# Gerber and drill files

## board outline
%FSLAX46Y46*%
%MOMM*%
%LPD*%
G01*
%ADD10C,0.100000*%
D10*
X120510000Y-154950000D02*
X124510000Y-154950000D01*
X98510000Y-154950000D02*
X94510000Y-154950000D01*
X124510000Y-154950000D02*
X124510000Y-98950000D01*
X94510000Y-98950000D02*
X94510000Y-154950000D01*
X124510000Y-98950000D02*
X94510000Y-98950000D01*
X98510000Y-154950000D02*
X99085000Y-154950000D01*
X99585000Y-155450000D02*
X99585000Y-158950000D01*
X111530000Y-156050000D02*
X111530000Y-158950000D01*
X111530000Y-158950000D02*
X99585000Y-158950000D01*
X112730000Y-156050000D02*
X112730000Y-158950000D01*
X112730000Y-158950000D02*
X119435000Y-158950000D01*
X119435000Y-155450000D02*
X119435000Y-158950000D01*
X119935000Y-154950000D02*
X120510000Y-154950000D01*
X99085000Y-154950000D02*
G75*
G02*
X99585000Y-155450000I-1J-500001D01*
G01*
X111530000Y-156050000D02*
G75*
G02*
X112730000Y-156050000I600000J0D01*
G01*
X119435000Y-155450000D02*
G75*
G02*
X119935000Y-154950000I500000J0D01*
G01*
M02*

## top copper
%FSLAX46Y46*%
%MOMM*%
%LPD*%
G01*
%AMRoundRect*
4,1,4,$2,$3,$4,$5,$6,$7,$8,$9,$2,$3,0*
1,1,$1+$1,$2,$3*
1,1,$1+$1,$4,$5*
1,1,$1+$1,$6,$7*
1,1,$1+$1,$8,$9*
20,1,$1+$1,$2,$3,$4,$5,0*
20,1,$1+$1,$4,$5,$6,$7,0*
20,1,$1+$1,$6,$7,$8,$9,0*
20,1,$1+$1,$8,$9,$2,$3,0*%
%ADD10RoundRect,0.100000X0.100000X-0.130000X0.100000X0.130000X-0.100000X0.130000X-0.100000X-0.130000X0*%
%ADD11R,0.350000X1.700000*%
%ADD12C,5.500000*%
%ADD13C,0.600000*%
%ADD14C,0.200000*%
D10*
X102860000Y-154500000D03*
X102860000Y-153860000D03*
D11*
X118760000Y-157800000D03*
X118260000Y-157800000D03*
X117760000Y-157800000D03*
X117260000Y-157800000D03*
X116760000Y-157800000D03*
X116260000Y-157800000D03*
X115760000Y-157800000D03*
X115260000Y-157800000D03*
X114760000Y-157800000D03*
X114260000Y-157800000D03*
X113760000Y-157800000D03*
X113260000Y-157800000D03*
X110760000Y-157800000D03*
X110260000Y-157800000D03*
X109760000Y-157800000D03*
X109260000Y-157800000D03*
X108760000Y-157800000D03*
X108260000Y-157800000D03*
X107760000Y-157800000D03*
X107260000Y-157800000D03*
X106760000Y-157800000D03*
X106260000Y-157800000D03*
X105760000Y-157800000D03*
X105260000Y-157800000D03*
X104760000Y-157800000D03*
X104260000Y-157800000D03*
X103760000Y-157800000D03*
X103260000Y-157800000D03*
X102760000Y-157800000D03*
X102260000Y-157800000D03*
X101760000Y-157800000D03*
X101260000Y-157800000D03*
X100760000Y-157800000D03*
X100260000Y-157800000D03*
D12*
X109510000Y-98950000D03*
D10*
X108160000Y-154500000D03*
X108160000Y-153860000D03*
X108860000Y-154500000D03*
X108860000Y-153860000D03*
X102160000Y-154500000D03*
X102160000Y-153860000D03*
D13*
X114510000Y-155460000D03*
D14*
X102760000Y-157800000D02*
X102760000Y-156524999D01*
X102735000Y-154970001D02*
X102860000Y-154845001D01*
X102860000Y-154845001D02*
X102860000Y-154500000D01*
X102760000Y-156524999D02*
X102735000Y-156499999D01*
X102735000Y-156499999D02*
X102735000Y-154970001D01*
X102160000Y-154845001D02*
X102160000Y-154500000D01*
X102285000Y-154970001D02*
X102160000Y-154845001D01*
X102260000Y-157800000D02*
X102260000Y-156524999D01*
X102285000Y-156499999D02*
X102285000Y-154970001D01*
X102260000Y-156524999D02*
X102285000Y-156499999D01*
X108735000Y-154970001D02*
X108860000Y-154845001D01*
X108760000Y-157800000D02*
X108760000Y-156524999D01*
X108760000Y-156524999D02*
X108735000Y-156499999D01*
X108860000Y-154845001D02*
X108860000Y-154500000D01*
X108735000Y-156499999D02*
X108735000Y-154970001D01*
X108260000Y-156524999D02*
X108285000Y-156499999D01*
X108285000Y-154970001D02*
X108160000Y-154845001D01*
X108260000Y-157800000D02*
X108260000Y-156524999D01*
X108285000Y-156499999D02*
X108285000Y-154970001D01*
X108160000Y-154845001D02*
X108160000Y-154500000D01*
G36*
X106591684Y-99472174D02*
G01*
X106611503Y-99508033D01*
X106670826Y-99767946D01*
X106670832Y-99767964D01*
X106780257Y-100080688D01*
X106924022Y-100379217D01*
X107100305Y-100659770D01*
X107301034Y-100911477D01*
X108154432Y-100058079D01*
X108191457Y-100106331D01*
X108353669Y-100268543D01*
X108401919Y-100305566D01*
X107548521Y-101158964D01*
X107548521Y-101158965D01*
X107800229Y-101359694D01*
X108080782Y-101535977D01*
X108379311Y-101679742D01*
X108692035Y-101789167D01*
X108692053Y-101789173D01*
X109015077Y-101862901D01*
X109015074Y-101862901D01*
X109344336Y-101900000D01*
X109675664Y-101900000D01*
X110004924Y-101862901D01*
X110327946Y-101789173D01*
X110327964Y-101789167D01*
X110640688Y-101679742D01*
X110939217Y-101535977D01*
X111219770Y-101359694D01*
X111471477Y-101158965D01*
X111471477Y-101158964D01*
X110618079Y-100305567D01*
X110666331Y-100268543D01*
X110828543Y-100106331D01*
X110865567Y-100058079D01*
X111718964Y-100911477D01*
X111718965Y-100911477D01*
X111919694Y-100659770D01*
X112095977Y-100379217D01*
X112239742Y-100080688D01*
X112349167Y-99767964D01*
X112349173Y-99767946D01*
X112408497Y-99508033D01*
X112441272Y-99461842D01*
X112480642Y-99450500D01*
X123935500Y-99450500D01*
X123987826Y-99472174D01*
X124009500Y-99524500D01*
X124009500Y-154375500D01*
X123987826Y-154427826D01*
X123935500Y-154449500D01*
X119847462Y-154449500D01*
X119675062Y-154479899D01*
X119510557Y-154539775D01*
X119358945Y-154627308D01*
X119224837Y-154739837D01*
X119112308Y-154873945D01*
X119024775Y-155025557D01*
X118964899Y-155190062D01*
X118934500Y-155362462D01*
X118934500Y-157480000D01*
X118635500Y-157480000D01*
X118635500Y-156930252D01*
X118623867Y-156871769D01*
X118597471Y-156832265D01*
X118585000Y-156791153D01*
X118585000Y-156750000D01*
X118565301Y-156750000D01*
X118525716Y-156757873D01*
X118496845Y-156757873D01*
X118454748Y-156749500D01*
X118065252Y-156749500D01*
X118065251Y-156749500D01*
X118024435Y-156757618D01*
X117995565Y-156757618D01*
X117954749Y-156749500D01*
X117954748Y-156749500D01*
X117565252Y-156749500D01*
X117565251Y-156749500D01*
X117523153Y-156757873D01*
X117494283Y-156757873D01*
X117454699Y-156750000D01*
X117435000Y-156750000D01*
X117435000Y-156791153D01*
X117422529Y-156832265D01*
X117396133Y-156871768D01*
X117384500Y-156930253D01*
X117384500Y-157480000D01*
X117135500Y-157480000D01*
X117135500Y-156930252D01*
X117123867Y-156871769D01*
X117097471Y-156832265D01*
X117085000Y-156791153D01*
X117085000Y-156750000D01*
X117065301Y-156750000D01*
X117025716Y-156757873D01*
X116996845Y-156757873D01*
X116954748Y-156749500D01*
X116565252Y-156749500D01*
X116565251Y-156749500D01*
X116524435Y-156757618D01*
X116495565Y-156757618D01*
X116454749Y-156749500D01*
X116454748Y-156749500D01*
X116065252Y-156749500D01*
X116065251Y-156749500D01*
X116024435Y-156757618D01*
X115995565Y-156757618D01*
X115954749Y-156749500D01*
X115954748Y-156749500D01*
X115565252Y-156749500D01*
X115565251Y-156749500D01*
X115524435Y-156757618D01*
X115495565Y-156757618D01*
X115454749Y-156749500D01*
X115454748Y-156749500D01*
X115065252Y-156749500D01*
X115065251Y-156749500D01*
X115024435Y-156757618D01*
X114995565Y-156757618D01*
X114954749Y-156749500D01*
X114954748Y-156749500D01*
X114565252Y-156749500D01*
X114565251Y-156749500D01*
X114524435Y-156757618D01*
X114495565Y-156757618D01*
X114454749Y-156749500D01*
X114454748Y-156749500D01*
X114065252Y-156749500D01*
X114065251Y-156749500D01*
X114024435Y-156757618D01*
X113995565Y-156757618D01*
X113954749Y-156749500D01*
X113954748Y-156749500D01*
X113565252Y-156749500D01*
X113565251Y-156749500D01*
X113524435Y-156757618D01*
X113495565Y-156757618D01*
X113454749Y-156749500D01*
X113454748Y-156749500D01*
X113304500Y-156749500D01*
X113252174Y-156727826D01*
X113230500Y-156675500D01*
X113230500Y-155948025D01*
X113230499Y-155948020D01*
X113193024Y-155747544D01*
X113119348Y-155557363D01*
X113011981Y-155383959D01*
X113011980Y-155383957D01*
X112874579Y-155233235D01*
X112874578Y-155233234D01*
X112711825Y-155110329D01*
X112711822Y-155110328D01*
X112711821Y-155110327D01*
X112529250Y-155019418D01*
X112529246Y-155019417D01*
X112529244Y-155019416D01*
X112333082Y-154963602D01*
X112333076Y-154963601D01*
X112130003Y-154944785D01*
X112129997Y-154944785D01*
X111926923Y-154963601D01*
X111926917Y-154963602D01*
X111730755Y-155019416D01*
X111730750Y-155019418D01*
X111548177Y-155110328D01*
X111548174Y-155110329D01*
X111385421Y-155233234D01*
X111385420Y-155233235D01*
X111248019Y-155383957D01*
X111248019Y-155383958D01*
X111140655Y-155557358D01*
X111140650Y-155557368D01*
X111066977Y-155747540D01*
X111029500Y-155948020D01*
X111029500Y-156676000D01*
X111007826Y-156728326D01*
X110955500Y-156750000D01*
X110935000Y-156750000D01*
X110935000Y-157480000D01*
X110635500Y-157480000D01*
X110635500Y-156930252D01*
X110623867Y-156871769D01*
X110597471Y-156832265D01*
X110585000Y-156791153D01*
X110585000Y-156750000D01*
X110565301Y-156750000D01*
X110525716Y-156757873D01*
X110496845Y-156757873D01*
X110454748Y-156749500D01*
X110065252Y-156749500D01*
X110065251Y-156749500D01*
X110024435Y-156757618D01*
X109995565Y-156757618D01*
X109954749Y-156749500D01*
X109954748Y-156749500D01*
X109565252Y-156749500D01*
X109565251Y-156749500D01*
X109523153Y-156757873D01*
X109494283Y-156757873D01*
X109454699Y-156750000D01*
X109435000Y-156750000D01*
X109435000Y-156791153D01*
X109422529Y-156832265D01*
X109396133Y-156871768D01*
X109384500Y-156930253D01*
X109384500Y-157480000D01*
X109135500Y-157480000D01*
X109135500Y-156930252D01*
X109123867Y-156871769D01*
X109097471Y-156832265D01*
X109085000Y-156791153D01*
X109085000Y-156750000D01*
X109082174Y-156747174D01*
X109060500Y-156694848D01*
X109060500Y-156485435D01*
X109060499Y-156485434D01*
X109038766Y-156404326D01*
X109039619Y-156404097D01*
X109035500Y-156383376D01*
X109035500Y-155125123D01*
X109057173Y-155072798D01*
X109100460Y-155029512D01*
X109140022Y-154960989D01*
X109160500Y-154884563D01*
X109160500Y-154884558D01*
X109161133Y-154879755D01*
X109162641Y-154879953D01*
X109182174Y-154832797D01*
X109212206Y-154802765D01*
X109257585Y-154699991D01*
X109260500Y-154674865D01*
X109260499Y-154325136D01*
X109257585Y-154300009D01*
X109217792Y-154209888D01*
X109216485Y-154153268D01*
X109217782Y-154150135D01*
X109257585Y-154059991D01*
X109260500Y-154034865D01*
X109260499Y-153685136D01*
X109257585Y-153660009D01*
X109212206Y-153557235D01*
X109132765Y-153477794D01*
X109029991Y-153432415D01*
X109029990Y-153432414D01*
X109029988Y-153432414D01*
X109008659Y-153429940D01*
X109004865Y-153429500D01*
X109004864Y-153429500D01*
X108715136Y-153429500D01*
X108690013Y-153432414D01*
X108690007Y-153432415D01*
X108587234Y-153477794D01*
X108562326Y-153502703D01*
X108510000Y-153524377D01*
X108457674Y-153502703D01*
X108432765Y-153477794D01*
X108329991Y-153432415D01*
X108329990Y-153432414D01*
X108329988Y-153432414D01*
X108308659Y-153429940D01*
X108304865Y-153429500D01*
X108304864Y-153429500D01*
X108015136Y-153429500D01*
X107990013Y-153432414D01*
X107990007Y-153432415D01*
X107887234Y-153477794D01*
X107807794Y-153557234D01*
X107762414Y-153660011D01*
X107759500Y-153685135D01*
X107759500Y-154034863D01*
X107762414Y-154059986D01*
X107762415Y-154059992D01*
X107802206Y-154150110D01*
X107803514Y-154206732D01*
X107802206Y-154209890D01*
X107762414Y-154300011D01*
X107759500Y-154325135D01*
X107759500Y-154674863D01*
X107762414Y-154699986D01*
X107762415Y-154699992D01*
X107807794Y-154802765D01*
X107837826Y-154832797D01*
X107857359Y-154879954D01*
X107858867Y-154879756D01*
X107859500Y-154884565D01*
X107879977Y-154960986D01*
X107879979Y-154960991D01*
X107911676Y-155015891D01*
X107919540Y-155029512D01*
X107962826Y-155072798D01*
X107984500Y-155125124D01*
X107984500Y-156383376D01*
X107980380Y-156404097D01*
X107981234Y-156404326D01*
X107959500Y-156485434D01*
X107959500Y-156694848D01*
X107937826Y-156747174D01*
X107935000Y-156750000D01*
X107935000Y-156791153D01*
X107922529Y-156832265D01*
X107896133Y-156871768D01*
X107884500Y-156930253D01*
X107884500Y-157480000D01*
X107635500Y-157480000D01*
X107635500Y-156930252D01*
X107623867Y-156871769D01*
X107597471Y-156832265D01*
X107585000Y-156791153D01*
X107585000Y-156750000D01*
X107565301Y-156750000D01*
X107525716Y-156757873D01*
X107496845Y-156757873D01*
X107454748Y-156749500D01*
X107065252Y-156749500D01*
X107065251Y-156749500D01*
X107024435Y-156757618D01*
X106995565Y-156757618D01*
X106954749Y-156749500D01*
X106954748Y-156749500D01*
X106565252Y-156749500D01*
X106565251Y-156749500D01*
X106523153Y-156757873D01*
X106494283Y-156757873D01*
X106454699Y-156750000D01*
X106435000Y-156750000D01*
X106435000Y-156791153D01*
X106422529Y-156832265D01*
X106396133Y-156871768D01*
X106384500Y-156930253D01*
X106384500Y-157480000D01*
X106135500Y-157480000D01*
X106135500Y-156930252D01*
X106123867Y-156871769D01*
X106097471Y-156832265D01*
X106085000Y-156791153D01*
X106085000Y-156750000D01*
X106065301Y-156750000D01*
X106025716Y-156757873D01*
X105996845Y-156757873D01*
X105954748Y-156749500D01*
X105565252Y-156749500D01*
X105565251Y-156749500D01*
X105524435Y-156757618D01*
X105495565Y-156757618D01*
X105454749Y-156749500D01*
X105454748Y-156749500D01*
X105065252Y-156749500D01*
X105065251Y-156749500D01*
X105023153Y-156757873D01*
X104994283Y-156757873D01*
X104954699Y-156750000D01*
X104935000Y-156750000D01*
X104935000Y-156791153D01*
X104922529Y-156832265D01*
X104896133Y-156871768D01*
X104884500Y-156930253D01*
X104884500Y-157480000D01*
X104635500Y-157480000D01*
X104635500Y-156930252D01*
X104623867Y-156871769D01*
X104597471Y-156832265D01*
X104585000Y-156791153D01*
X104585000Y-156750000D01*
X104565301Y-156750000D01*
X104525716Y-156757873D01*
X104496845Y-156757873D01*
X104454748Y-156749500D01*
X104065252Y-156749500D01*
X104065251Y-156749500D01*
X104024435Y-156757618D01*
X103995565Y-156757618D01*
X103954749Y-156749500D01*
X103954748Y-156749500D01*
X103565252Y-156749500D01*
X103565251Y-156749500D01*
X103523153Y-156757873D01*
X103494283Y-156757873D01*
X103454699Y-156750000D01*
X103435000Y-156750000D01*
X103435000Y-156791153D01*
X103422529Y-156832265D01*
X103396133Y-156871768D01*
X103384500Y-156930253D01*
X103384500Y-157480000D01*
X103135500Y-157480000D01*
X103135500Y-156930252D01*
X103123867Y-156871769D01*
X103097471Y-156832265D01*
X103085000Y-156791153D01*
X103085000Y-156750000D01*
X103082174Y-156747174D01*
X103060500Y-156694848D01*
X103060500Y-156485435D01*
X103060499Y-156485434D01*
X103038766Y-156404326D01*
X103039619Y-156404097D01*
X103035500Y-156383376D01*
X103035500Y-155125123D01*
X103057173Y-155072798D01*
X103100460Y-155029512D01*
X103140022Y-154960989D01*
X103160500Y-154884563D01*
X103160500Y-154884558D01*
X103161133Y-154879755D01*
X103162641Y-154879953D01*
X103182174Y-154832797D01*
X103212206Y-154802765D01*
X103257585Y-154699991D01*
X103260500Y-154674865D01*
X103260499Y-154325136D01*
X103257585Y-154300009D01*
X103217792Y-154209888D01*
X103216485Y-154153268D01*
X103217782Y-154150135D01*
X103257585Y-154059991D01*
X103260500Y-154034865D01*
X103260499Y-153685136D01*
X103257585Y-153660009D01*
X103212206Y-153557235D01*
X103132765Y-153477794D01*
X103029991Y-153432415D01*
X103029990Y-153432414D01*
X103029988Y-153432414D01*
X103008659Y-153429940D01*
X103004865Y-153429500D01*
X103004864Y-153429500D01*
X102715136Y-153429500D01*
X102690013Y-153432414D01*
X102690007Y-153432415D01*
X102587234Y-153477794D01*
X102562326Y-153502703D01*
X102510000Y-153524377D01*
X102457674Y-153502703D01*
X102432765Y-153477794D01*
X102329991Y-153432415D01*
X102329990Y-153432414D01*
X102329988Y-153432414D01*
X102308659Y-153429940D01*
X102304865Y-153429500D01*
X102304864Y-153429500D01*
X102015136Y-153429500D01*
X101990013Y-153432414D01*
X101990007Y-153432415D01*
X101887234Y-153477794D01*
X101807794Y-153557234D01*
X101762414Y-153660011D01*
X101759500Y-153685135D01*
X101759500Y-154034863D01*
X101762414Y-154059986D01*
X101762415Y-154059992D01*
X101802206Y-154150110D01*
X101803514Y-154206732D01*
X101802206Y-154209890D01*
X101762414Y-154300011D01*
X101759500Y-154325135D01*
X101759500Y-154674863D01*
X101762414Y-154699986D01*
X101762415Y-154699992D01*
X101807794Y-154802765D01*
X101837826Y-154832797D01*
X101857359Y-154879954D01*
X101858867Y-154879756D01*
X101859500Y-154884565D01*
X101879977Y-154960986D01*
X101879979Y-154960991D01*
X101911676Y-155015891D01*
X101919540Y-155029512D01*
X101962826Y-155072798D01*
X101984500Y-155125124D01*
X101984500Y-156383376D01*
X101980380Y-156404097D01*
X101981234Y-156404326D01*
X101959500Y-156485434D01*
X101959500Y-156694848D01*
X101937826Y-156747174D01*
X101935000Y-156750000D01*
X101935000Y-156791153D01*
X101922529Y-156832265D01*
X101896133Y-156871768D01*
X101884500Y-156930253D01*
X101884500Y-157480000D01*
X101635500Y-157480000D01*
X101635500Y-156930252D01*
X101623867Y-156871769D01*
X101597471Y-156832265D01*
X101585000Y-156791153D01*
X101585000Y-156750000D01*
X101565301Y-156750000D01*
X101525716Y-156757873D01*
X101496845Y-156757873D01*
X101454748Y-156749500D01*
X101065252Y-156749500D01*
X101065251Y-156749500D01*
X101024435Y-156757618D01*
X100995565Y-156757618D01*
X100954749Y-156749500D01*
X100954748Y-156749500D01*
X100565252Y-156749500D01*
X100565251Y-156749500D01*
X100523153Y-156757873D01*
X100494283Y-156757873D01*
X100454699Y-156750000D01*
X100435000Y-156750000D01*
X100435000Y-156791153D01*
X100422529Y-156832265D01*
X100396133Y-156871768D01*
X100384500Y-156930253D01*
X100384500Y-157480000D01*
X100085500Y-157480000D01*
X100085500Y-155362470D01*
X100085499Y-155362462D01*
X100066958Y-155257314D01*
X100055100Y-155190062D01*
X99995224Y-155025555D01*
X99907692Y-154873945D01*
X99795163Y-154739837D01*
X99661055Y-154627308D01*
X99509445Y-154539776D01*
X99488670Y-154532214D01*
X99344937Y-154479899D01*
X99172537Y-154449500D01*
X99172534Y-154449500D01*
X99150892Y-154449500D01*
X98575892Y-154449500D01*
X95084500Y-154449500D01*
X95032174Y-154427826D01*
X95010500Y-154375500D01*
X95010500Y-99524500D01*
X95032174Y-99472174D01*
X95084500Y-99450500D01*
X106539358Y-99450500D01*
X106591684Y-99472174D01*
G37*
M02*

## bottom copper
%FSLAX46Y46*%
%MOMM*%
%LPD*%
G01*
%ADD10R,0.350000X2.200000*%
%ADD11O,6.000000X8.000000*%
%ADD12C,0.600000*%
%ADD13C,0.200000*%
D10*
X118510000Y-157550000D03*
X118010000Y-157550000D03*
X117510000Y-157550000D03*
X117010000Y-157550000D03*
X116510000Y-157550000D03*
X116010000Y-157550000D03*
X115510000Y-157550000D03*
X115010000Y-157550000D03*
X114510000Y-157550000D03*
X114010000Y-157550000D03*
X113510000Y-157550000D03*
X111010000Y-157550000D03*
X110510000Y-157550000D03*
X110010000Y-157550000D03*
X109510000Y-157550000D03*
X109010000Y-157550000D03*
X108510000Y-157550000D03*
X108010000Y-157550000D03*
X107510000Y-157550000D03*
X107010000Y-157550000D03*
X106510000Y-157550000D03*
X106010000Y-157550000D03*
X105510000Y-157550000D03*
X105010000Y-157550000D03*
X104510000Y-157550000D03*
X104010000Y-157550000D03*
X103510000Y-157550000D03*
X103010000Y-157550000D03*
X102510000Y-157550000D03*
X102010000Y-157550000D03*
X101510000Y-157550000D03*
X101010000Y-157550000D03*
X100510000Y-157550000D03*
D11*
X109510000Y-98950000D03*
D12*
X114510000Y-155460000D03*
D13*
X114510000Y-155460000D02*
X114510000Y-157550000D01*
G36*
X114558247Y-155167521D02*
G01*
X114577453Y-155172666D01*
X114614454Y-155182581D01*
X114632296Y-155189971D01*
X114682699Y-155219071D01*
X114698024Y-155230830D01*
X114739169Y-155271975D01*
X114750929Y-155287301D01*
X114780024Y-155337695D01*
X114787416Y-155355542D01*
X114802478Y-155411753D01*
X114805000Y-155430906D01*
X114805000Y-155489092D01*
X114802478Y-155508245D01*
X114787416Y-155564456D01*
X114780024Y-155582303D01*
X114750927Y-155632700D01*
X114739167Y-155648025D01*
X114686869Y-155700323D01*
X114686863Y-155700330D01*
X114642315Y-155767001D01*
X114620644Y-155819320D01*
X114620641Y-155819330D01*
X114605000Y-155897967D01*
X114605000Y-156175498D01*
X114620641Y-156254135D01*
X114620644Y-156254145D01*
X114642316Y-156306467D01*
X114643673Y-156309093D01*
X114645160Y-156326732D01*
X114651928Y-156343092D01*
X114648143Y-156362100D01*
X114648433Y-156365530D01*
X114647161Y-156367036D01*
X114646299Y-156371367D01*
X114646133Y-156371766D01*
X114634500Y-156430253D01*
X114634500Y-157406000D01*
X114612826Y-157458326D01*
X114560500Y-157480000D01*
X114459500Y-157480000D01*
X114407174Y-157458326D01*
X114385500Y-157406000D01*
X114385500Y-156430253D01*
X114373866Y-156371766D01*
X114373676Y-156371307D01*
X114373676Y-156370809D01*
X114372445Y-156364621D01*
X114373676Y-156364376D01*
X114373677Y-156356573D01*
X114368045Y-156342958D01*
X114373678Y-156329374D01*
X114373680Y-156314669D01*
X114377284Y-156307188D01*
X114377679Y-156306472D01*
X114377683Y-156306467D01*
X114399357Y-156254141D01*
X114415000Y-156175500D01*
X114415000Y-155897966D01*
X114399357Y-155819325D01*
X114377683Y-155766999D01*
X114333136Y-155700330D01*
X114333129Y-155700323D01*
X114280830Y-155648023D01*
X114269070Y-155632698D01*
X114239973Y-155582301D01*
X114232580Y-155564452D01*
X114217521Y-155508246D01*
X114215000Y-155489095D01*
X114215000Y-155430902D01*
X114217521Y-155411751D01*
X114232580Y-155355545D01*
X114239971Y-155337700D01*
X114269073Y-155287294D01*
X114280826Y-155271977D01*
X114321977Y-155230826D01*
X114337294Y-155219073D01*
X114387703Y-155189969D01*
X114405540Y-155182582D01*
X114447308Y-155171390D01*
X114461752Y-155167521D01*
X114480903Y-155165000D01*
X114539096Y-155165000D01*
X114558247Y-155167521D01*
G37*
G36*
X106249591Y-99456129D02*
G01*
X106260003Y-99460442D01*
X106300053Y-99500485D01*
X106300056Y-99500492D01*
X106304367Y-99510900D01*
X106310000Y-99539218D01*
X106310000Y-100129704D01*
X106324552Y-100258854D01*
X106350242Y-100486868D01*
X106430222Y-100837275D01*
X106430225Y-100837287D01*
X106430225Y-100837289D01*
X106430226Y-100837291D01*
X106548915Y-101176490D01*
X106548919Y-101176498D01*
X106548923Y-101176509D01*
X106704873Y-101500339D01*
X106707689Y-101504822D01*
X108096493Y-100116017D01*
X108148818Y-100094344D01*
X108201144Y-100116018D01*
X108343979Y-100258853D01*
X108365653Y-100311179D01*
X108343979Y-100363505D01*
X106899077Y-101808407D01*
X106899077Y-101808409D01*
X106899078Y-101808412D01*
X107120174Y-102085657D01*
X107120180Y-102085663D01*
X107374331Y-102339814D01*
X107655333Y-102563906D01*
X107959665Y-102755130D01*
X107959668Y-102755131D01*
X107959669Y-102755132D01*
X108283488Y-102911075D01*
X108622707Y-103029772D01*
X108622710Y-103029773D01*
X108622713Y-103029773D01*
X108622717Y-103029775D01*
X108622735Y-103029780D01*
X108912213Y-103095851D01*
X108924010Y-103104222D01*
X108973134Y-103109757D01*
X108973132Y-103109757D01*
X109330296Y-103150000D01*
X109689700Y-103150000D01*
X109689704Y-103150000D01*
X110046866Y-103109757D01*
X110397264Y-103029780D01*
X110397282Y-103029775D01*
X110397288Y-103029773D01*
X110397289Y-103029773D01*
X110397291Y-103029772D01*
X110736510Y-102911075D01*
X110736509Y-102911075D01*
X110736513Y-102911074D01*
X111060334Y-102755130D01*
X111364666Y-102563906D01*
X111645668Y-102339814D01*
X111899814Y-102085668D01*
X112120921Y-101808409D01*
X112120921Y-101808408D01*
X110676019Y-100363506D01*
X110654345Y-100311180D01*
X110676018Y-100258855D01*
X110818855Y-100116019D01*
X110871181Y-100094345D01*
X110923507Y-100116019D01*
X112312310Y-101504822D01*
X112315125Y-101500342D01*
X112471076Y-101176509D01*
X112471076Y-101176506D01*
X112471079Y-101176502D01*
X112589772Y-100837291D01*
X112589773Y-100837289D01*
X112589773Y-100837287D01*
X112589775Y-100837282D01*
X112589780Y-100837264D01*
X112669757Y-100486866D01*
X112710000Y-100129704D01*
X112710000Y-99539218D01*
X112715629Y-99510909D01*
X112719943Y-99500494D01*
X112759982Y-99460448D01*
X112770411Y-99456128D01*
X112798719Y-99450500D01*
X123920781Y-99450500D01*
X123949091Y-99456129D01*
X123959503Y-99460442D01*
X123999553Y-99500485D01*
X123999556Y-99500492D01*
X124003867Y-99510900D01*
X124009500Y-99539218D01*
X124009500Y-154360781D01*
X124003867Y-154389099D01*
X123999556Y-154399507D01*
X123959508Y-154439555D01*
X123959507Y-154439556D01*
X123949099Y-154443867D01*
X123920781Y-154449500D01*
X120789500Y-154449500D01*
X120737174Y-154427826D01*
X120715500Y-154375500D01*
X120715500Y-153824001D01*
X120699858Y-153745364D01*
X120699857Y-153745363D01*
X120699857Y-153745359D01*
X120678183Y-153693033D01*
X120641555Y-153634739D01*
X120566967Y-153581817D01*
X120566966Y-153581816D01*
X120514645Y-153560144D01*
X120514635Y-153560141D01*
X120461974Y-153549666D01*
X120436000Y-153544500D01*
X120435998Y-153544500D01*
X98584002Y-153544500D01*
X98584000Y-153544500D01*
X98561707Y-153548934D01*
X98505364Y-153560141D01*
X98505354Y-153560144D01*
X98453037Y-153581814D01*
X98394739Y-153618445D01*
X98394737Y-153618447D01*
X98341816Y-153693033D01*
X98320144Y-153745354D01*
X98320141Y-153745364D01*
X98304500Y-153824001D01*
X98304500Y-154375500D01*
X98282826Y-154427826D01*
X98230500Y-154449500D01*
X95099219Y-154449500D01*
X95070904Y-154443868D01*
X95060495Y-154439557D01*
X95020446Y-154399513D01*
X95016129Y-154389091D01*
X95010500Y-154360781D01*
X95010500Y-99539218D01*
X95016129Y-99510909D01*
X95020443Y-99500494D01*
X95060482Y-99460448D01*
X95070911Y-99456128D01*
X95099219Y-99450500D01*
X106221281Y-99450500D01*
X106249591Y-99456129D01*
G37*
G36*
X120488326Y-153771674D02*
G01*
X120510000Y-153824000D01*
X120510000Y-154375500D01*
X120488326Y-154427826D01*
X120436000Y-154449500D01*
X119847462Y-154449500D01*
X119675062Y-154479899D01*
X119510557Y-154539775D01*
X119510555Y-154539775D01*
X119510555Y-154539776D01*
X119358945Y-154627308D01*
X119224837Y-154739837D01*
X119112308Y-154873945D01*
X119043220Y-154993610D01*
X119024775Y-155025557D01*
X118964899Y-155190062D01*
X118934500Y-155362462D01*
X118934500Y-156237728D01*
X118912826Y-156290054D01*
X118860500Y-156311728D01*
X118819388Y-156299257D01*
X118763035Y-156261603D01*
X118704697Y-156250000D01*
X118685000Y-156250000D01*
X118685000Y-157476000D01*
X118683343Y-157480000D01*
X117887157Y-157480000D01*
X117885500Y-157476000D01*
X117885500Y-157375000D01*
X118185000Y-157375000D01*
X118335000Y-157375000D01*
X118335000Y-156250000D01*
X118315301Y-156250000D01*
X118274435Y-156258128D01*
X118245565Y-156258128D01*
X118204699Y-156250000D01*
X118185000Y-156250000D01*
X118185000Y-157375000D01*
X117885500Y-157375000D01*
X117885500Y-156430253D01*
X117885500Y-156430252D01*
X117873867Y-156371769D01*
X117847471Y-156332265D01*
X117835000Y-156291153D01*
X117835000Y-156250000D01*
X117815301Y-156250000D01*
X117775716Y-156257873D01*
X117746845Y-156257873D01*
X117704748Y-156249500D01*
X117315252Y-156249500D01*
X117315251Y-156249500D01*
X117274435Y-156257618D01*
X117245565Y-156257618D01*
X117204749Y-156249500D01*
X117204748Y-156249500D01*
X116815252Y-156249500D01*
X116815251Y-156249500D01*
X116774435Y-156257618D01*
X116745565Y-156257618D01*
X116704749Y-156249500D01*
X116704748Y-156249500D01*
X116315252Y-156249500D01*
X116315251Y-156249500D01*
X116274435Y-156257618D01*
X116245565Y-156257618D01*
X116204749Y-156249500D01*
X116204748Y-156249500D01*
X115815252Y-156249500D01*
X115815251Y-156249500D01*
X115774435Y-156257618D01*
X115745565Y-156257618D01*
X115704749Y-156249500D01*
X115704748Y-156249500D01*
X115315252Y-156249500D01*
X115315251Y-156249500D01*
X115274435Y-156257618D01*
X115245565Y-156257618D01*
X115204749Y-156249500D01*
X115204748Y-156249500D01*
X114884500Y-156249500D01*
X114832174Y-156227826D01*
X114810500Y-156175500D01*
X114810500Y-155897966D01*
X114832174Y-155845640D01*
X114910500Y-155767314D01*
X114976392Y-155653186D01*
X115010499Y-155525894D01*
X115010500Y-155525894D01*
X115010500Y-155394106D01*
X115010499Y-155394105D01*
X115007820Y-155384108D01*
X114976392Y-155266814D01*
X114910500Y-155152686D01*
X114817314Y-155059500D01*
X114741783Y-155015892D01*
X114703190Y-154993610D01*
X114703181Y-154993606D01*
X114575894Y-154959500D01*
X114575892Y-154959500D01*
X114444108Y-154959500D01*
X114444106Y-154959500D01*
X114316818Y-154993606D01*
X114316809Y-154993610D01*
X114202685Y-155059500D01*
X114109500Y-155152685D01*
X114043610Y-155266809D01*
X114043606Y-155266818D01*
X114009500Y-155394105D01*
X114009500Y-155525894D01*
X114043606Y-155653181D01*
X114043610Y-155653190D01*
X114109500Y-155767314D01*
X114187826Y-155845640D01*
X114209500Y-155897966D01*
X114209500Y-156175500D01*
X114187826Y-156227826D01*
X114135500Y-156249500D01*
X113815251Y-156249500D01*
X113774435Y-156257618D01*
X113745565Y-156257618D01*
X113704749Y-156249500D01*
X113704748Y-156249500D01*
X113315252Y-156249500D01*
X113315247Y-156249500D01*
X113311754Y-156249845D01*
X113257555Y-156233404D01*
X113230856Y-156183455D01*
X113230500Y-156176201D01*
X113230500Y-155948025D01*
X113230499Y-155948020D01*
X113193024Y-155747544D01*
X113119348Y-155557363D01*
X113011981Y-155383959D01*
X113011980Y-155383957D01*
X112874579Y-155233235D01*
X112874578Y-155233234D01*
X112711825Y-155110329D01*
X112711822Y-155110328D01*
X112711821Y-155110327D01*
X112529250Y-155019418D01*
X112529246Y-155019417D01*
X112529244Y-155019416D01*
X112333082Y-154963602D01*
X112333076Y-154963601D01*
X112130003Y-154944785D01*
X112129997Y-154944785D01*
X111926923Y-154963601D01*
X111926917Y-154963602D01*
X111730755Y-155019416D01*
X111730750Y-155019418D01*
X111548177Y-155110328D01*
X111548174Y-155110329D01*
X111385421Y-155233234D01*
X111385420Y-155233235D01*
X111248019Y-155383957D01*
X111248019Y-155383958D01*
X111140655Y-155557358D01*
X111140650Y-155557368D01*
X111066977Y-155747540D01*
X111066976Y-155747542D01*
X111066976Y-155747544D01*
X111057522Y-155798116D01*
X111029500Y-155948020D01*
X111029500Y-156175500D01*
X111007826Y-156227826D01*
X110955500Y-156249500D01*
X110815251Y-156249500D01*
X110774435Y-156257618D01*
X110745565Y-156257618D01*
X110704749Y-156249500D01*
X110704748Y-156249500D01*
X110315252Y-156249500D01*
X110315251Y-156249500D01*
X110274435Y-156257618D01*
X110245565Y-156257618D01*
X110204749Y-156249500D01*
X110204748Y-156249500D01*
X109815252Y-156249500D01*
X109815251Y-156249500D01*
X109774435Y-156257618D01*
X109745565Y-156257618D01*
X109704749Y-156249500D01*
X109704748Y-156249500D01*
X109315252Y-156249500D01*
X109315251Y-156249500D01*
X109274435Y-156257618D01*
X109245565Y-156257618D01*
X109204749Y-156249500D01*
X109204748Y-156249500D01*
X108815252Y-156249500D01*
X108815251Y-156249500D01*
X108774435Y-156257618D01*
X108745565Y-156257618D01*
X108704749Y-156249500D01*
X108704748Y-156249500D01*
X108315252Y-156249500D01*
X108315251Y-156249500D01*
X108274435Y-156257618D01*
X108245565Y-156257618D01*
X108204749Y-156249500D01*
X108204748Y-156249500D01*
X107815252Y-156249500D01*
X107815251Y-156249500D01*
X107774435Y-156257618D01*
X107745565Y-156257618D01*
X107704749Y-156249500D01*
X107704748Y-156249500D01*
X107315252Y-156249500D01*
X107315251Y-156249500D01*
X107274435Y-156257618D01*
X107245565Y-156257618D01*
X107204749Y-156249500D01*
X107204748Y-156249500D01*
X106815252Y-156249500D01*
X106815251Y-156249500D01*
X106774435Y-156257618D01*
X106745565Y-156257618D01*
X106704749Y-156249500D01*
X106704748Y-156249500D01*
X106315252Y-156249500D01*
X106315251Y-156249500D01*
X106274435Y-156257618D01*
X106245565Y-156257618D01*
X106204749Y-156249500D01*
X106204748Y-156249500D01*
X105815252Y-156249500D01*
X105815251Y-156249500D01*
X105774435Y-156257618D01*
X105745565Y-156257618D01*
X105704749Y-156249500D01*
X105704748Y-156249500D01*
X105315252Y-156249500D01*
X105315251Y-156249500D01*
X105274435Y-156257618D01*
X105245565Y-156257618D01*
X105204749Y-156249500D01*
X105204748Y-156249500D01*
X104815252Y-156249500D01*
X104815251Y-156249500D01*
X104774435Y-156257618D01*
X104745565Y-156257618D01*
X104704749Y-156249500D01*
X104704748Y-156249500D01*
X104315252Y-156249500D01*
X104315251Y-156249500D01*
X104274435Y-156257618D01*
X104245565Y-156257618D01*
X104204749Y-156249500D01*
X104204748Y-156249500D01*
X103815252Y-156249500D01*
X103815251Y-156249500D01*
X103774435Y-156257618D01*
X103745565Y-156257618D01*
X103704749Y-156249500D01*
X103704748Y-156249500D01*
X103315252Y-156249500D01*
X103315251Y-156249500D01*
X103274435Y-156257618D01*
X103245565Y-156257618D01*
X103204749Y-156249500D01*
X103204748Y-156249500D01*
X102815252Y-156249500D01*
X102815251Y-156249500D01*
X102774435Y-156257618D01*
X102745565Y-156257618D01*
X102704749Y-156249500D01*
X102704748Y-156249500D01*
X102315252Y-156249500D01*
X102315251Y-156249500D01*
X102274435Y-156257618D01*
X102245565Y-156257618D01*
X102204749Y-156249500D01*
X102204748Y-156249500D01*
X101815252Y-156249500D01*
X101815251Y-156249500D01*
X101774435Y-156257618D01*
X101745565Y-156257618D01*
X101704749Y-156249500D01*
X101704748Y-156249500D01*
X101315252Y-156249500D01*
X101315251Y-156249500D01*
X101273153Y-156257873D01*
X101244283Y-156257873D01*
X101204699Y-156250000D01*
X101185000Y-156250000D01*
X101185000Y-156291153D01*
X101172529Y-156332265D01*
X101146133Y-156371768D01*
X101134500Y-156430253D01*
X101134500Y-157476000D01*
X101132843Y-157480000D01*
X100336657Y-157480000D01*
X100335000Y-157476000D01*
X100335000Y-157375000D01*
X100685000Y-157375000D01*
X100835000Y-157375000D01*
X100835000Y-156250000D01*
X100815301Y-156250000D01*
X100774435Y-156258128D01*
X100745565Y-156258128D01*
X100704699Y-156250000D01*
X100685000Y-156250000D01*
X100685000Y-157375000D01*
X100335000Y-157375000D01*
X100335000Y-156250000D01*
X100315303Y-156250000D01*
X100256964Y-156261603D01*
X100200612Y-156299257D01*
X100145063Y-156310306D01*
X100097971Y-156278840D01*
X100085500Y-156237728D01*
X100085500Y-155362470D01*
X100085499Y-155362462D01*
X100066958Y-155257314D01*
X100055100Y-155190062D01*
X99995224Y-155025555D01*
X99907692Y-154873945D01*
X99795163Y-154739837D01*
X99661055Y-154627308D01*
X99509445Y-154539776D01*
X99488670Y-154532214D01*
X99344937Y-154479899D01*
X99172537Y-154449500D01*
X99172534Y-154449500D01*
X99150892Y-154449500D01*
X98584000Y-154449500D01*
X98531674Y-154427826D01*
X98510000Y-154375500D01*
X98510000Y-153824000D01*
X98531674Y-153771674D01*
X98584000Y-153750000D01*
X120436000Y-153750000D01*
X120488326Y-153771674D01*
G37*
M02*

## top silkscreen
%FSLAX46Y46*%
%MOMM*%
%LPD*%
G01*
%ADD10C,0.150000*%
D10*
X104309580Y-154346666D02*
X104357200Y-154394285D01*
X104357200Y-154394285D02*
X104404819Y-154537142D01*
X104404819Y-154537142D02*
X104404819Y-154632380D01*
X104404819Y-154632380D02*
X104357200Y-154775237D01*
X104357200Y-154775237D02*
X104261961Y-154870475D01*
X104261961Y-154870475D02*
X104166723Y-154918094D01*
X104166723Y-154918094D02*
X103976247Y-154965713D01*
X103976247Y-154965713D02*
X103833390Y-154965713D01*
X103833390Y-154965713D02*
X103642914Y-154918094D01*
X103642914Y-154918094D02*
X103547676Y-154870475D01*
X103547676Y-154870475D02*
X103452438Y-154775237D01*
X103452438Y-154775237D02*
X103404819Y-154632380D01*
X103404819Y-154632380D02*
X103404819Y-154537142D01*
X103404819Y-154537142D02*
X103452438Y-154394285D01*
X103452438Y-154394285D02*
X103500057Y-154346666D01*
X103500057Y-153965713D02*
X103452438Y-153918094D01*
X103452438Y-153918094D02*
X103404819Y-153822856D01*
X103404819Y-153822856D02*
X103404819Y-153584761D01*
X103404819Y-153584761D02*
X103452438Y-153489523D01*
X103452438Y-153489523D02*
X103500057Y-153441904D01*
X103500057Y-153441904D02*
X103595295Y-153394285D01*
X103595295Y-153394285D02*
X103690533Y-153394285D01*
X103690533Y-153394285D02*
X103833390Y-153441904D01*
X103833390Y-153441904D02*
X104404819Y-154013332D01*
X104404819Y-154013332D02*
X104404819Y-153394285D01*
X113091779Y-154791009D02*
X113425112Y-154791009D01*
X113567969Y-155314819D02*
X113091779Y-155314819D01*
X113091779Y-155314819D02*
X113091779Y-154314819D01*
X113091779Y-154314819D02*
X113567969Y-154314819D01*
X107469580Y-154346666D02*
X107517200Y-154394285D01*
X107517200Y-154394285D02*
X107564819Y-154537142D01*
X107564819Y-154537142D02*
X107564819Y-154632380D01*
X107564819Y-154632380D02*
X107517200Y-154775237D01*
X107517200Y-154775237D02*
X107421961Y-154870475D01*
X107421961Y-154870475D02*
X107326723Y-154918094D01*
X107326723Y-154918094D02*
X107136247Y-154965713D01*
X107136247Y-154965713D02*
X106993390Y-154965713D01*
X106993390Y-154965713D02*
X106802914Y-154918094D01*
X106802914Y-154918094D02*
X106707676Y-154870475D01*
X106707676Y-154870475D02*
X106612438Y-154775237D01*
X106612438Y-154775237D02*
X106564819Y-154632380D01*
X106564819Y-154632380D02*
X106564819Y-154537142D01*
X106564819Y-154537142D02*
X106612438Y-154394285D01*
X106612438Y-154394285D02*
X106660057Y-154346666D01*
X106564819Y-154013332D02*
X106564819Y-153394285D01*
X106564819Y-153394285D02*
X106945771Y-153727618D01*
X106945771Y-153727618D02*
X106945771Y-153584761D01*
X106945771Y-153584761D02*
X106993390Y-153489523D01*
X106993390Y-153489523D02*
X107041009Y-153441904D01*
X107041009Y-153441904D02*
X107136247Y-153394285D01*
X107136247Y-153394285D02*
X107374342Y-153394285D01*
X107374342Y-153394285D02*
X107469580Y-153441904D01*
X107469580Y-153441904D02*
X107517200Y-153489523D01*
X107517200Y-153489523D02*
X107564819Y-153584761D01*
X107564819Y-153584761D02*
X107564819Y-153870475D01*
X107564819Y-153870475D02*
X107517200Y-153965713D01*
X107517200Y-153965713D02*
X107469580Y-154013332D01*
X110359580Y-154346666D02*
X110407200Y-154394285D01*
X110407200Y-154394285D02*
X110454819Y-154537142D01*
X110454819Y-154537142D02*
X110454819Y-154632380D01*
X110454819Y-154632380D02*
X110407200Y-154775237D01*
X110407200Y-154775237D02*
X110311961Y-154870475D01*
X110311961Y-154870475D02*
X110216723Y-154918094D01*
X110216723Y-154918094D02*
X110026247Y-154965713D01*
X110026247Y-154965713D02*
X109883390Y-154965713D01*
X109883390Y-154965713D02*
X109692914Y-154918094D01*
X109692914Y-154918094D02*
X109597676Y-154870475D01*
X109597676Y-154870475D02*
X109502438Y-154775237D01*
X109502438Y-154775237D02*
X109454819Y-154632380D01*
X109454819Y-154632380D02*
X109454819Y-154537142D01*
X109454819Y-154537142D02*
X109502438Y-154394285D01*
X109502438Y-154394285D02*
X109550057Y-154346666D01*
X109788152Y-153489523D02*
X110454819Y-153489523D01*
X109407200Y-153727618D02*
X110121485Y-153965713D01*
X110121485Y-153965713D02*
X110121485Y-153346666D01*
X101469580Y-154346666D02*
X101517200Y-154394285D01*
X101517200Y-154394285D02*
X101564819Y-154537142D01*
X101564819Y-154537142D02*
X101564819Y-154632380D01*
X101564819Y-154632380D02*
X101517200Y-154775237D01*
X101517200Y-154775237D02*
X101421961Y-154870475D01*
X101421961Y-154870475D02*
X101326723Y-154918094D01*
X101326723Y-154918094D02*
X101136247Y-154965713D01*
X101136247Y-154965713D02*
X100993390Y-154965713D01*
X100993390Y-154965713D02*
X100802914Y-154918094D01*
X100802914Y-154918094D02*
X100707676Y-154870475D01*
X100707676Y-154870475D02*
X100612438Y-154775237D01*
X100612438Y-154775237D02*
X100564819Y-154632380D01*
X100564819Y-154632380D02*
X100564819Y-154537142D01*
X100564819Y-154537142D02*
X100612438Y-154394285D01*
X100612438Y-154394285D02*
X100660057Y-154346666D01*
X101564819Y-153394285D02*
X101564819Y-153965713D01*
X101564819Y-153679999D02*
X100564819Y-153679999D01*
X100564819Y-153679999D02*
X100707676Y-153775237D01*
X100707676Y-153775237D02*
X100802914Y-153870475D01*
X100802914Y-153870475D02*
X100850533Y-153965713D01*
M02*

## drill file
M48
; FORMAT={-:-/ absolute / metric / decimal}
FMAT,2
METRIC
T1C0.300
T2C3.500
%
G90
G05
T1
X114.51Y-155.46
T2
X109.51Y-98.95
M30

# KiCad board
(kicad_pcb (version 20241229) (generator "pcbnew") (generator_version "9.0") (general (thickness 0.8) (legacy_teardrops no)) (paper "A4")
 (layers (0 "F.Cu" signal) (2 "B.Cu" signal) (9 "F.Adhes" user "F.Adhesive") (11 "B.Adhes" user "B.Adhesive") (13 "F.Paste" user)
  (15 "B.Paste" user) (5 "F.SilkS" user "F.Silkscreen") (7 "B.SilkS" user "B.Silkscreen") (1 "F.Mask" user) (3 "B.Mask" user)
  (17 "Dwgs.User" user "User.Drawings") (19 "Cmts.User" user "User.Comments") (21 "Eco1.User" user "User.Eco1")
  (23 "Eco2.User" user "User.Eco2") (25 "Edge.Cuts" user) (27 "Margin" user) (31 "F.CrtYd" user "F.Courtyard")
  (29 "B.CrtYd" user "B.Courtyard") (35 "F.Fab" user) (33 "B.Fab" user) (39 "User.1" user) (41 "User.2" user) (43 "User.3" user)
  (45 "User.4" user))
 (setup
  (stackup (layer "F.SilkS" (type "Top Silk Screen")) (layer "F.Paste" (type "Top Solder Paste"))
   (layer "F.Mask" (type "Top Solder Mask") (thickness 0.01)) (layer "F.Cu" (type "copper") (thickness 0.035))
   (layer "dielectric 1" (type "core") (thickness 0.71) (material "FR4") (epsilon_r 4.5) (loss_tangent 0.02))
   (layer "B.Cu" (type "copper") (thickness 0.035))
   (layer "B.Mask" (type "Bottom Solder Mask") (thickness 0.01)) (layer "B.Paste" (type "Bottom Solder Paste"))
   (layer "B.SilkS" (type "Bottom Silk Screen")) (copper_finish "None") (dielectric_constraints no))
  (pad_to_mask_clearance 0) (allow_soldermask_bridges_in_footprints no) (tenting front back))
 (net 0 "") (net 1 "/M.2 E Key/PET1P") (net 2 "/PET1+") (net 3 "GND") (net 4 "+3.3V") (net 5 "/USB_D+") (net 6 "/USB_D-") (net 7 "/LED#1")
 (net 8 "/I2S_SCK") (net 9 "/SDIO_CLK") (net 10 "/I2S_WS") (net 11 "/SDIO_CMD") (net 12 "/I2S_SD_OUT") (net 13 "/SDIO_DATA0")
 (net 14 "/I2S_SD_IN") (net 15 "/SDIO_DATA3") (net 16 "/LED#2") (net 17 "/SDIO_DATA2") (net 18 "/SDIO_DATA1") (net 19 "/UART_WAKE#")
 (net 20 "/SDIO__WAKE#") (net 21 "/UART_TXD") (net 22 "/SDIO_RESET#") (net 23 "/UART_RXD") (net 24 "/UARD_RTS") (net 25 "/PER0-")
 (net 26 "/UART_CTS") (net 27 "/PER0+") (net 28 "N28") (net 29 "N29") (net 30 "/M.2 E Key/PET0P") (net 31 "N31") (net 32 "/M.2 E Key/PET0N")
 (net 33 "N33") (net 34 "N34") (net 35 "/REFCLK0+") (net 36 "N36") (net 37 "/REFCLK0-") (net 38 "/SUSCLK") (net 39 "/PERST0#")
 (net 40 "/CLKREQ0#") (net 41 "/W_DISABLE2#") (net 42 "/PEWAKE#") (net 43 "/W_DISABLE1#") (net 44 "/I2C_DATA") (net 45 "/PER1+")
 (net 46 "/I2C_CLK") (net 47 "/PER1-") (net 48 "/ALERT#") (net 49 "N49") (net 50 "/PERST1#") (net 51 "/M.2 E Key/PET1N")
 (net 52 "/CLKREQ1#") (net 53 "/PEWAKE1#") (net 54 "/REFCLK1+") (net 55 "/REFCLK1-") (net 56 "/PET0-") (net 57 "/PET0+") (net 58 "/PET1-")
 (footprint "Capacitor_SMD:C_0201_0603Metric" (layer "F.Cu") (at 102.86 154.18 90)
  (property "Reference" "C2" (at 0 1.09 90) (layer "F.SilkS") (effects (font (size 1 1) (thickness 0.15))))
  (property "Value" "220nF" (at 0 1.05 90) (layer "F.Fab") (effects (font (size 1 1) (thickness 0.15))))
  (pad "" smd roundrect (at -0.345 0 90) (size 0.318 0.36) (layers "F.Paste") (roundrect_rratio 0.25))
  (pad "" smd roundrect (at 0.345 0 90) (size 0.318 0.36) (layers "F.Paste") (roundrect_rratio 0.25))
  (pad "1" smd roundrect (at -0.32 0 90) (size 0.46 0.4) (layers "F.Cu" "F.Mask") (roundrect_rratio 0.25) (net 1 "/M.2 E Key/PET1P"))
  (pad "2" smd roundrect (at 0.32 0 90) (size 0.46 0.4) (layers "F.Cu" "F.Mask") (roundrect_rratio 0.25) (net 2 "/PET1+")))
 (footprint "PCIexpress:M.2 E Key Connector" (layer "F.Cu") (at 109.51 157.84)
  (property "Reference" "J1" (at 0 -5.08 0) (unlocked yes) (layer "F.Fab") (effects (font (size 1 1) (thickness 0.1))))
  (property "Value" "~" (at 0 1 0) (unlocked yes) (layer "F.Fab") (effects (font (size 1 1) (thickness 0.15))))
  (fp_line (start -11 -2.89) (end -10.425 -2.89) (stroke (width 0.1) (type default)) (layer "Edge.Cuts") (net 1))
  (fp_line (start -9.925 -2.39) (end -9.925 1.11) (stroke (width 0.1) (type default)) (layer "Edge.Cuts") (net 1))
  (fp_line (start 2.02 -1.79) (end 2.02 1.11) (stroke (width 0.1) (type default)) (layer "Edge.Cuts") (net 1))
  (fp_line (start 2.02 1.11) (end -9.925 1.11) (stroke (width 0.1) (type default)) (layer "Edge.Cuts") (net 1))
  (fp_line (start 3.22 -1.79) (end 3.22 1.11) (stroke (width 0.1) (type default)) (layer "Edge.Cuts") (net 1))
  (fp_line (start 3.22 1.11) (end 9.925 1.11) (stroke (width 0.1) (type default)) (layer "Edge.Cuts") (net 1))
  (fp_line (start 9.925 -2.39) (end 9.925 1.11) (stroke (width 0.1) (type default)) (layer "Edge.Cuts") (net 1))
  (fp_line (start 10.425 -2.89) (end 11 -2.89) (stroke (width 0.1) (type default)) (layer "Edge.Cuts") (net 1))
  (fp_arc (start -10.425 -2.89) (mid -10.071447 -2.743553) (end -9.925 -2.39) (stroke (width 0.1) (type default)) (layer "Edge.Cuts")
   (net 1))
  (fp_arc (start 2.02 -1.79) (mid 2.62 -2.39) (end 3.22 -1.79) (stroke (width 0.1) (type default)) (layer "Edge.Cuts") (net 1))
  (fp_arc (start 9.925 -2.39) (mid 10.071447 -2.743553) (end 10.425 -2.89) (stroke (width 0.1) (type default)) (layer "Edge.Cuts") (net 1))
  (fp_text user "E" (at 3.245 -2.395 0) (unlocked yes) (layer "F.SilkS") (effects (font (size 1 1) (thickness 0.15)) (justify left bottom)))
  (pad "1" smd rect (at 9.25 -0.04 180) (size 0.35 1.7) (layers "F.Cu") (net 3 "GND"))
  (pad "2" smd rect (at 9 -0.29 180) (size 0.35 2.2) (layers "B.Cu") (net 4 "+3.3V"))
  (pad "3" smd rect (at 8.75 -0.04 180) (size 0.35 1.7) (layers "F.Cu") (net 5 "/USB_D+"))
  (pad "4" smd rect (at 8.5 -0.29 180) (size 0.35 2.2) (layers "B.Cu") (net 4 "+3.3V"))
  (pad "5" smd rect (at 8.25 -0.04 180) (size 0.35 1.7) (layers "F.Cu") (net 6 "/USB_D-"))
  (pad "6" smd rect (at 8 -0.29 180) (size 0.35 2.2) (layers "B.Cu") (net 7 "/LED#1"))
  (pad "7" smd rect (at 7.75 -0.04 180) (size 0.35 1.7) (layers "F.Cu") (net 3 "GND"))
  (pad "8" smd rect (at 7.5 -0.29 180) (size 0.35 2.2) (layers "B.Cu") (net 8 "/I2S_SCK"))
  (pad "9" smd rect (at 7.25 -0.04 180) (size 0.35 1.7) (layers "F.Cu") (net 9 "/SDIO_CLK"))
  (pad "10" smd rect (at 7 -0.29 180) (size 0.35 2.2) (layers "B.Cu") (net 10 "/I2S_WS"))
  (pad "11" smd rect (at 6.75 -0.04 180) (size 0.35 1.7) (layers "F.Cu") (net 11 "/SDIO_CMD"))
  (pad "12" smd rect (at 6.5 -0.29 180) (size 0.35 2.2) (layers "B.Cu") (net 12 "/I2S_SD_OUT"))
  (pad "13" smd rect (at 6.25 -0.04 180) (size 0.35 1.7) (layers "F.Cu") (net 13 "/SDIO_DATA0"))
  (pad "14" smd rect (at 6 -0.29 180) (size 0.35 2.2) (layers "B.Cu") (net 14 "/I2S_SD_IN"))
  (pad "15" smd rect (at 5.75 -0.04 180) (size 0.35 1.7) (layers "F.Cu") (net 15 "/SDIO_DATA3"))
  (pad "16" smd rect (at 5.5 -0.29 180) (size 0.35 2.2) (layers "B.Cu") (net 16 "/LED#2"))
  (pad "17" smd rect (at 5.25 -0.04 180) (size 0.35 1.7) (layers "F.Cu") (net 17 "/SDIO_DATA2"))
  (pad "18" smd rect (at 5 -0.29 180) (size 0.35 2.2) (layers "B.Cu") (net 3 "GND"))
  (pad "19" smd rect (at 4.75 -0.04 180) (size 0.35 1.7) (layers "F.Cu") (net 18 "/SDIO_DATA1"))
  (pad "20" smd rect (at 4.5 -0.29 180) (size 0.35 2.2) (layers "B.Cu") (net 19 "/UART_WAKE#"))
  (pad "21" smd rect (at 4.25 -0.04 180) (size 0.35 1.7) (layers "F.Cu") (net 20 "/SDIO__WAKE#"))
  (pad "22" smd rect (at 4 -0.29 180) (size 0.35 2.2) (layers "B.Cu") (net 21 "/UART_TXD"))
  (pad "23" smd rect (at 3.75 -0.04 180) (size 0.35 1.7) (layers "F.Cu") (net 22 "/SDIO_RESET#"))
  (pad "32" smd rect (at 1.5 -0.29 180) (size 0.35 2.2) (layers "B.Cu") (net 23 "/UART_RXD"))
  (pad "33" smd rect (at 1.25 -0.04 180) (size 0.35 1.7) (layers "F.Cu") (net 3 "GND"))
  (pad "34" smd rect (at 1 -0.29 180) (size 0.35 2.2) (layers "B.Cu") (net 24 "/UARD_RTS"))
  (pad "35" smd rect (at 0.75 -0.04 180) (size 0.35 1.7) (layers "F.Cu") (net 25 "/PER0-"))
  (pad "36" smd rect (at 0.5 -0.29 180) (size 0.35 2.2) (layers "B.Cu") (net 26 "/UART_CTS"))
  (pad "37" smd rect (at 0.25 -0.04 180) (size 0.35 1.7) (layers "F.Cu") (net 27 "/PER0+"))
  (pad "38" smd rect (at 0 -0.29 180) (size 0.35 2.2) (layers "B.Cu") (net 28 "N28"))
  (pad "39" smd rect (at -0.25 -0.04 180) (size 0.35 1.7) (layers "F.Cu") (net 3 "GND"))
  (pad "40" smd rect (at -0.5 -0.29 180) (size 0.35 2.2) (layers "B.Cu") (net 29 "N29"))
  (pad "41" smd rect (at -0.75 -0.04 180) (size 0.35 1.7) (layers "F.Cu") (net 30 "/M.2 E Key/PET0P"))
  (pad "42" smd rect (at -1 -0.29 180) (size 0.35 2.2) (layers "B.Cu") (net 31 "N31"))
  (pad "43" smd rect (at -1.25 -0.04 180) (size 0.35 1.7) (layers "F.Cu") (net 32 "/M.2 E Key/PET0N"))
  (pad "44" smd rect (at -1.5 -0.29 180) (size 0.35 2.2) (layers "B.Cu") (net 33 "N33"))
  (pad "45" smd rect (at -1.75 -0.04 180) (size 0.35 1.7) (layers "F.Cu") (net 3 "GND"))
  (pad "46" smd rect (at -2 -0.29 180) (size 0.35 2.2) (layers "B.Cu") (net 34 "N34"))
  (pad "47" smd rect (at -2.25 -0.04 180) (size 0.35 1.7) (layers "F.Cu") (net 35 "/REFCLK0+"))
  (pad "48" smd rect (at -2.5 -0.29 180) (size 0.35 2.2) (layers "B.Cu") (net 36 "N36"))
  (pad "49" smd rect (at -2.75 -0.04 180) (size 0.35 1.7) (layers "F.Cu") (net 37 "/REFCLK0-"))
  (pad "50" smd rect (at -3 -0.29 180) (size 0.35 2.2) (layers "B.Cu") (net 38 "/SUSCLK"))
  (pad "51" smd rect (at -3.25 -0.04 180) (size 0.35 1.7) (layers "F.Cu") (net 3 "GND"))
  (pad "52" smd rect (at -3.5 -0.29 180) (size 0.35 2.2) (layers "B.Cu") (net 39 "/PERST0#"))
  (pad "53" smd rect (at -3.75 -0.04 180) (size 0.35 1.7) (layers "F.Cu") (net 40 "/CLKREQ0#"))
  (pad "54" smd rect (at -4 -0.29 180) (size 0.35 2.2) (layers "B.Cu") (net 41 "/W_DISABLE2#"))
  (pad "55" smd rect (at -4.25 -0.04 180) (size 0.35 1.7) (layers "F.Cu") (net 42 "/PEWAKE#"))
  (pad "56" smd rect (at -4.5 -0.29 180) (size 0.35 2.2) (layers "B.Cu") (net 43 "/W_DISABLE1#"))
  (pad "57" smd rect (at -4.75 -0.04 180) (size 0.35 1.7) (layers "F.Cu") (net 3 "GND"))
  (pad "58" smd rect (at -5 -0.29 180) (size 0.35 2.2) (layers "B.Cu") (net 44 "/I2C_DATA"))
  (pad "59" smd rect (at -5.25 -0.04 180) (size 0.35 1.7) (layers "F.Cu") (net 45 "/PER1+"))
  (pad "60" smd rect (at -5.5 -0.29 180) (size 0.35 2.2) (layers "B.Cu") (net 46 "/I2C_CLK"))
  (pad "61" smd rect (at -5.75 -0.04 180) (size 0.35 1.7) (layers "F.Cu") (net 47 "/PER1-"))
  (pad "62" smd rect (at -6 -0.29 180) (size 0.35 2.2) (layers "B.Cu") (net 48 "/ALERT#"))
  (pad "63" smd rect (at -6.25 -0.04 180) (size 0.35 1.7) (layers "F.Cu") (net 3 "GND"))
  (pad "64" smd rect (at -6.5 -0.29 180) (size 0.35 2.2) (layers "B.Cu") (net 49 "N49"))
  (pad "65" smd rect (at -6.75 -0.04 180) (size 0.35 1.7) (layers "F.Cu") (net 1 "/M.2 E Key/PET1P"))
  (pad "66" smd rect (at -7 -0.29 180) (size 0.35 2.2) (layers "B.Cu") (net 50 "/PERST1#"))
  (pad "67" smd rect (at -7.25 -0.04 180) (size 0.35 1.7) (layers "F.Cu") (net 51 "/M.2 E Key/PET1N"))
  (pad "68" smd rect (at -7.5 -0.29 180) (size 0.35 2.2) (layers "B.Cu") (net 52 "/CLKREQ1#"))
  (pad "69" smd rect (at -7.75 -0.04 180) (size 0.35 1.7) (layers "F.Cu") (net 3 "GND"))
  (pad "70" smd rect (at -8 -0.29 180) (size 0.35 2.2) (layers "B.Cu") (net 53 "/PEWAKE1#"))
  (pad "71" smd rect (at -8.25 -0.04 180) (size 0.35 1.7) (layers "F.Cu") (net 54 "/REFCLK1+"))
  (pad "72" smd rect (at -8.5 -0.29 180) (size 0.35 2.2) (layers "B.Cu") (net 4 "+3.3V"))
  (pad "73" smd rect (at -8.75 -0.04 180) (size 0.35 1.7) (layers "F.Cu") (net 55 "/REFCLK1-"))
  (pad "74" smd rect (at -9 -0.29 180) (size 0.35 2.2) (layers "B.Cu") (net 4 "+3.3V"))
  (pad "75" smd rect (at -9.25 -0.04 180) (size 0.35 1.7) (layers "F.Cu") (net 3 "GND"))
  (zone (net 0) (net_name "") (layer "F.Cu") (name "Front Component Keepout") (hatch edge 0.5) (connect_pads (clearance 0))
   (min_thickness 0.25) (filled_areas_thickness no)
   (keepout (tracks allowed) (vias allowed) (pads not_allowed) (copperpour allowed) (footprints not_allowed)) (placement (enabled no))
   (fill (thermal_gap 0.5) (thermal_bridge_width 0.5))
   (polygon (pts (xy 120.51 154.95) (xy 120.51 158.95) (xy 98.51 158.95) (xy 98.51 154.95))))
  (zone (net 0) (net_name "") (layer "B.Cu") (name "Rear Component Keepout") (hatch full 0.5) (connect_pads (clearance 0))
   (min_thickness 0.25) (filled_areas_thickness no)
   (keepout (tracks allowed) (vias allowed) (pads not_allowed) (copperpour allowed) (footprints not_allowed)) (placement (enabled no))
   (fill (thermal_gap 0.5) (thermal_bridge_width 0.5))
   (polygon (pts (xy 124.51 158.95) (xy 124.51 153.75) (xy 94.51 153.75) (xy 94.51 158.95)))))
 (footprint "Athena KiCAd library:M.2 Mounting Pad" (layer "F.Cu") (at 109.51 98.95)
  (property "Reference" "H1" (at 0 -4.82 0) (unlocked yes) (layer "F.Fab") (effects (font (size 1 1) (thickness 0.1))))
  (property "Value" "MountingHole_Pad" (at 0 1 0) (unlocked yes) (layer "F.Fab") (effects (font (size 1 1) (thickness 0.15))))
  (pad "1" thru_hole circle (at 0 0) (size 5.5 5.5) (drill 3.5) (layers "*.Cu" "*.Mask") (remove_unused_layers no) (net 3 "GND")
   (padstack (mode front_inner_back)
    (layer "Inner" (shape circle) (size 5.5 5.5) (zone_connect -1))
    (layer "B.Cu" (shape oval) (size 6 8) (thermal_bridge_angle 45) (zone_connect -1)))))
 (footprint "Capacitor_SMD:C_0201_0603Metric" (layer "F.Cu") (at 108.16 154.18 90)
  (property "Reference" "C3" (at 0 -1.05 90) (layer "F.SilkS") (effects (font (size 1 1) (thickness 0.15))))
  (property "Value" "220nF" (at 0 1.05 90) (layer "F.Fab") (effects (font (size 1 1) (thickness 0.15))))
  (pad "" smd roundrect (at -0.345 0 90) (size 0.318 0.36) (layers "F.Paste") (roundrect_rratio 0.25))
  (pad "" smd roundrect (at 0.345 0 90) (size 0.318 0.36) (layers "F.Paste") (roundrect_rratio 0.25))
  (pad "1" smd roundrect (at -0.32 0 90) (size 0.46 0.4) (layers "F.Cu" "F.Mask") (roundrect_rratio 0.25) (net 32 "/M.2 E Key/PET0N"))
  (pad "2" smd roundrect (at 0.32 0 90) (size 0.46 0.4) (layers "F.Cu" "F.Mask") (roundrect_rratio 0.25) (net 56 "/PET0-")))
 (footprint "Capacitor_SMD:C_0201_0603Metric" (layer "F.Cu") (at 108.86 154.18 90)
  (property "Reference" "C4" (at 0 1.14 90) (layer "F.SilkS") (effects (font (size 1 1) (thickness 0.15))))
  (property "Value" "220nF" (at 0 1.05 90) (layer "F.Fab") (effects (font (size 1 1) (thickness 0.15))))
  (pad "" smd roundrect (at -0.345 0 90) (size 0.318 0.36) (layers "F.Paste") (roundrect_rratio 0.25))
  (pad "" smd roundrect (at 0.345 0 90) (size 0.318 0.36) (layers "F.Paste") (roundrect_rratio 0.25))
  (pad "1" smd roundrect (at -0.32 0 90) (size 0.46 0.4) (layers "F.Cu" "F.Mask") (roundrect_rratio 0.25) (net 30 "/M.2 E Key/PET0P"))
  (pad "2" smd roundrect (at 0.32 0 90) (size 0.46 0.4) (layers "F.Cu" "F.Mask") (roundrect_rratio 0.25) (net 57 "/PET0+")))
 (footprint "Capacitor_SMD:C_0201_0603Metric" (layer "F.Cu") (at 102.16 154.18 90)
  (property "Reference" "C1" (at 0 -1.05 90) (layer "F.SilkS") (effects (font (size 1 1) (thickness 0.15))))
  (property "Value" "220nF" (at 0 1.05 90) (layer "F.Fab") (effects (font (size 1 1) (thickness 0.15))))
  (pad "" smd roundrect (at -0.345 0 90) (size 0.318 0.36) (layers "F.Paste") (roundrect_rratio 0.25))
  (pad "" smd roundrect (at 0.345 0 90) (size 0.318 0.36) (layers "F.Paste") (roundrect_rratio 0.25))
  (pad "1" smd roundrect (at -0.32 0 90) (size 0.46 0.4) (layers "F.Cu" "F.Mask") (roundrect_rratio 0.25) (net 51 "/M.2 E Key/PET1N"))
  (pad "2" smd roundrect (at 0.32 0 90) (size 0.46 0.4) (layers "F.Cu" "F.Mask") (roundrect_rratio 0.25) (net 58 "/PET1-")))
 (gr_line (start 120.51 154.95) (end 124.51 154.95) (stroke (width 0.1) (type default)) (layer "Edge.Cuts"))
 (gr_line (start 98.51 154.95) (end 94.51 154.95) (stroke (width 0.1) (type default)) (layer "Edge.Cuts"))
 (gr_line (start 124.51 154.95) (end 124.51 98.95) (stroke (width 0.1) (type default)) (layer "Edge.Cuts"))
 (gr_line (start 94.51 98.95) (end 94.51 154.95) (stroke (width 0.1) (type default)) (layer "Edge.Cuts"))
 (gr_line (start 124.51 98.95) (end 94.51 98.95) (stroke (width 0.1) (type default)) (layer "Edge.Cuts"))
 (segment (start 102.76 157.8) (end 102.76 156.524999) (width 0.2) (layer "F.Cu") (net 1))
 (segment (start 102.735 154.970001) (end 102.86 154.845001) (width 0.2) (layer "F.Cu") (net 1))
 (segment (start 102.86 154.845001) (end 102.86 154.5) (width 0.2) (layer "F.Cu") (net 1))
 (segment (start 102.76 156.524999) (end 102.735 156.499999) (width 0.2) (layer "F.Cu") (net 1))
 (segment (start 102.735 156.499999) (end 102.735 154.970001) (width 0.2) (layer "F.Cu") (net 1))
 (segment (start 102.16 154.845001) (end 102.16 154.5) (width 0.2) (layer "F.Cu") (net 51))
 (segment (start 102.285 154.970001) (end 102.16 154.845001) (width 0.2) (layer "F.Cu") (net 51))
 (segment (start 102.26 157.8) (end 102.26 156.524999) (width 0.2) (layer "F.Cu") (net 51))
 (segment (start 102.285 156.499999) (end 102.285 154.970001) (width 0.2) (layer "F.Cu") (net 51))
 (segment (start 102.26 156.524999) (end 102.285 156.499999) (width 0.2) (layer "F.Cu") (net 51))
 (segment (start 108.735 154.970001) (end 108.86 154.845001) (width 0.2) (layer "F.Cu") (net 30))
 (segment (start 108.76 157.8) (end 108.76 156.524999) (width 0.2) (layer "F.Cu") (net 30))
 (segment (start 108.76 156.524999) (end 108.735 156.499999) (width 0.2) (layer "F.Cu") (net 30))
 (segment (start 108.86 154.845001) (end 108.86 154.5) (width 0.2) (layer "F.Cu") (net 30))
 (segment (start 108.735 156.499999) (end 108.735 154.970001) (width 0.2) (layer "F.Cu") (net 30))
 (segment (start 108.26 156.524999) (end 108.285 156.499999) (width 0.2) (layer "F.Cu") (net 32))
 (segment (start 108.285 154.970001) (end 108.16 154.845001) (width 0.2) (layer "F.Cu") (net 32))
 (segment (start 108.26 157.8) (end 108.26 156.524999) (width 0.2) (layer "F.Cu") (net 32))
 (segment (start 108.285 156.499999) (end 108.285 154.970001) (width 0.2) (layer "F.Cu") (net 32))
 (segment (start 108.16 154.845001) (end 108.16 154.5) (width 0.2) (layer "F.Cu") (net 32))
 (via (at 114.51 155.46) (size 0.6) (drill 0.3) (layers "F.Cu" "B.Cu") (free yes) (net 3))
 (segment (start 114.51 155.46) (end 114.51 157.55) (width 0.2) (layer "B.Cu") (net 3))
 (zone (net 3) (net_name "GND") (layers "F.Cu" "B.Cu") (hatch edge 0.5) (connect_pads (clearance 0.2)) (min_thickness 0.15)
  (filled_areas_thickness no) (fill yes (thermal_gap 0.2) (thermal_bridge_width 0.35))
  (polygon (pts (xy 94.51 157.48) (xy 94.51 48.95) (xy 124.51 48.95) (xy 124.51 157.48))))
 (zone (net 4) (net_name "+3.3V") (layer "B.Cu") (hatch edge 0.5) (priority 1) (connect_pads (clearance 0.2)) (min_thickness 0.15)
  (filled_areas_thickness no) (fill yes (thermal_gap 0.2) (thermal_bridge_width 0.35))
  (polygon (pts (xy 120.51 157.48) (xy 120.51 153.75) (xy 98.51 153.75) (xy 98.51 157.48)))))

